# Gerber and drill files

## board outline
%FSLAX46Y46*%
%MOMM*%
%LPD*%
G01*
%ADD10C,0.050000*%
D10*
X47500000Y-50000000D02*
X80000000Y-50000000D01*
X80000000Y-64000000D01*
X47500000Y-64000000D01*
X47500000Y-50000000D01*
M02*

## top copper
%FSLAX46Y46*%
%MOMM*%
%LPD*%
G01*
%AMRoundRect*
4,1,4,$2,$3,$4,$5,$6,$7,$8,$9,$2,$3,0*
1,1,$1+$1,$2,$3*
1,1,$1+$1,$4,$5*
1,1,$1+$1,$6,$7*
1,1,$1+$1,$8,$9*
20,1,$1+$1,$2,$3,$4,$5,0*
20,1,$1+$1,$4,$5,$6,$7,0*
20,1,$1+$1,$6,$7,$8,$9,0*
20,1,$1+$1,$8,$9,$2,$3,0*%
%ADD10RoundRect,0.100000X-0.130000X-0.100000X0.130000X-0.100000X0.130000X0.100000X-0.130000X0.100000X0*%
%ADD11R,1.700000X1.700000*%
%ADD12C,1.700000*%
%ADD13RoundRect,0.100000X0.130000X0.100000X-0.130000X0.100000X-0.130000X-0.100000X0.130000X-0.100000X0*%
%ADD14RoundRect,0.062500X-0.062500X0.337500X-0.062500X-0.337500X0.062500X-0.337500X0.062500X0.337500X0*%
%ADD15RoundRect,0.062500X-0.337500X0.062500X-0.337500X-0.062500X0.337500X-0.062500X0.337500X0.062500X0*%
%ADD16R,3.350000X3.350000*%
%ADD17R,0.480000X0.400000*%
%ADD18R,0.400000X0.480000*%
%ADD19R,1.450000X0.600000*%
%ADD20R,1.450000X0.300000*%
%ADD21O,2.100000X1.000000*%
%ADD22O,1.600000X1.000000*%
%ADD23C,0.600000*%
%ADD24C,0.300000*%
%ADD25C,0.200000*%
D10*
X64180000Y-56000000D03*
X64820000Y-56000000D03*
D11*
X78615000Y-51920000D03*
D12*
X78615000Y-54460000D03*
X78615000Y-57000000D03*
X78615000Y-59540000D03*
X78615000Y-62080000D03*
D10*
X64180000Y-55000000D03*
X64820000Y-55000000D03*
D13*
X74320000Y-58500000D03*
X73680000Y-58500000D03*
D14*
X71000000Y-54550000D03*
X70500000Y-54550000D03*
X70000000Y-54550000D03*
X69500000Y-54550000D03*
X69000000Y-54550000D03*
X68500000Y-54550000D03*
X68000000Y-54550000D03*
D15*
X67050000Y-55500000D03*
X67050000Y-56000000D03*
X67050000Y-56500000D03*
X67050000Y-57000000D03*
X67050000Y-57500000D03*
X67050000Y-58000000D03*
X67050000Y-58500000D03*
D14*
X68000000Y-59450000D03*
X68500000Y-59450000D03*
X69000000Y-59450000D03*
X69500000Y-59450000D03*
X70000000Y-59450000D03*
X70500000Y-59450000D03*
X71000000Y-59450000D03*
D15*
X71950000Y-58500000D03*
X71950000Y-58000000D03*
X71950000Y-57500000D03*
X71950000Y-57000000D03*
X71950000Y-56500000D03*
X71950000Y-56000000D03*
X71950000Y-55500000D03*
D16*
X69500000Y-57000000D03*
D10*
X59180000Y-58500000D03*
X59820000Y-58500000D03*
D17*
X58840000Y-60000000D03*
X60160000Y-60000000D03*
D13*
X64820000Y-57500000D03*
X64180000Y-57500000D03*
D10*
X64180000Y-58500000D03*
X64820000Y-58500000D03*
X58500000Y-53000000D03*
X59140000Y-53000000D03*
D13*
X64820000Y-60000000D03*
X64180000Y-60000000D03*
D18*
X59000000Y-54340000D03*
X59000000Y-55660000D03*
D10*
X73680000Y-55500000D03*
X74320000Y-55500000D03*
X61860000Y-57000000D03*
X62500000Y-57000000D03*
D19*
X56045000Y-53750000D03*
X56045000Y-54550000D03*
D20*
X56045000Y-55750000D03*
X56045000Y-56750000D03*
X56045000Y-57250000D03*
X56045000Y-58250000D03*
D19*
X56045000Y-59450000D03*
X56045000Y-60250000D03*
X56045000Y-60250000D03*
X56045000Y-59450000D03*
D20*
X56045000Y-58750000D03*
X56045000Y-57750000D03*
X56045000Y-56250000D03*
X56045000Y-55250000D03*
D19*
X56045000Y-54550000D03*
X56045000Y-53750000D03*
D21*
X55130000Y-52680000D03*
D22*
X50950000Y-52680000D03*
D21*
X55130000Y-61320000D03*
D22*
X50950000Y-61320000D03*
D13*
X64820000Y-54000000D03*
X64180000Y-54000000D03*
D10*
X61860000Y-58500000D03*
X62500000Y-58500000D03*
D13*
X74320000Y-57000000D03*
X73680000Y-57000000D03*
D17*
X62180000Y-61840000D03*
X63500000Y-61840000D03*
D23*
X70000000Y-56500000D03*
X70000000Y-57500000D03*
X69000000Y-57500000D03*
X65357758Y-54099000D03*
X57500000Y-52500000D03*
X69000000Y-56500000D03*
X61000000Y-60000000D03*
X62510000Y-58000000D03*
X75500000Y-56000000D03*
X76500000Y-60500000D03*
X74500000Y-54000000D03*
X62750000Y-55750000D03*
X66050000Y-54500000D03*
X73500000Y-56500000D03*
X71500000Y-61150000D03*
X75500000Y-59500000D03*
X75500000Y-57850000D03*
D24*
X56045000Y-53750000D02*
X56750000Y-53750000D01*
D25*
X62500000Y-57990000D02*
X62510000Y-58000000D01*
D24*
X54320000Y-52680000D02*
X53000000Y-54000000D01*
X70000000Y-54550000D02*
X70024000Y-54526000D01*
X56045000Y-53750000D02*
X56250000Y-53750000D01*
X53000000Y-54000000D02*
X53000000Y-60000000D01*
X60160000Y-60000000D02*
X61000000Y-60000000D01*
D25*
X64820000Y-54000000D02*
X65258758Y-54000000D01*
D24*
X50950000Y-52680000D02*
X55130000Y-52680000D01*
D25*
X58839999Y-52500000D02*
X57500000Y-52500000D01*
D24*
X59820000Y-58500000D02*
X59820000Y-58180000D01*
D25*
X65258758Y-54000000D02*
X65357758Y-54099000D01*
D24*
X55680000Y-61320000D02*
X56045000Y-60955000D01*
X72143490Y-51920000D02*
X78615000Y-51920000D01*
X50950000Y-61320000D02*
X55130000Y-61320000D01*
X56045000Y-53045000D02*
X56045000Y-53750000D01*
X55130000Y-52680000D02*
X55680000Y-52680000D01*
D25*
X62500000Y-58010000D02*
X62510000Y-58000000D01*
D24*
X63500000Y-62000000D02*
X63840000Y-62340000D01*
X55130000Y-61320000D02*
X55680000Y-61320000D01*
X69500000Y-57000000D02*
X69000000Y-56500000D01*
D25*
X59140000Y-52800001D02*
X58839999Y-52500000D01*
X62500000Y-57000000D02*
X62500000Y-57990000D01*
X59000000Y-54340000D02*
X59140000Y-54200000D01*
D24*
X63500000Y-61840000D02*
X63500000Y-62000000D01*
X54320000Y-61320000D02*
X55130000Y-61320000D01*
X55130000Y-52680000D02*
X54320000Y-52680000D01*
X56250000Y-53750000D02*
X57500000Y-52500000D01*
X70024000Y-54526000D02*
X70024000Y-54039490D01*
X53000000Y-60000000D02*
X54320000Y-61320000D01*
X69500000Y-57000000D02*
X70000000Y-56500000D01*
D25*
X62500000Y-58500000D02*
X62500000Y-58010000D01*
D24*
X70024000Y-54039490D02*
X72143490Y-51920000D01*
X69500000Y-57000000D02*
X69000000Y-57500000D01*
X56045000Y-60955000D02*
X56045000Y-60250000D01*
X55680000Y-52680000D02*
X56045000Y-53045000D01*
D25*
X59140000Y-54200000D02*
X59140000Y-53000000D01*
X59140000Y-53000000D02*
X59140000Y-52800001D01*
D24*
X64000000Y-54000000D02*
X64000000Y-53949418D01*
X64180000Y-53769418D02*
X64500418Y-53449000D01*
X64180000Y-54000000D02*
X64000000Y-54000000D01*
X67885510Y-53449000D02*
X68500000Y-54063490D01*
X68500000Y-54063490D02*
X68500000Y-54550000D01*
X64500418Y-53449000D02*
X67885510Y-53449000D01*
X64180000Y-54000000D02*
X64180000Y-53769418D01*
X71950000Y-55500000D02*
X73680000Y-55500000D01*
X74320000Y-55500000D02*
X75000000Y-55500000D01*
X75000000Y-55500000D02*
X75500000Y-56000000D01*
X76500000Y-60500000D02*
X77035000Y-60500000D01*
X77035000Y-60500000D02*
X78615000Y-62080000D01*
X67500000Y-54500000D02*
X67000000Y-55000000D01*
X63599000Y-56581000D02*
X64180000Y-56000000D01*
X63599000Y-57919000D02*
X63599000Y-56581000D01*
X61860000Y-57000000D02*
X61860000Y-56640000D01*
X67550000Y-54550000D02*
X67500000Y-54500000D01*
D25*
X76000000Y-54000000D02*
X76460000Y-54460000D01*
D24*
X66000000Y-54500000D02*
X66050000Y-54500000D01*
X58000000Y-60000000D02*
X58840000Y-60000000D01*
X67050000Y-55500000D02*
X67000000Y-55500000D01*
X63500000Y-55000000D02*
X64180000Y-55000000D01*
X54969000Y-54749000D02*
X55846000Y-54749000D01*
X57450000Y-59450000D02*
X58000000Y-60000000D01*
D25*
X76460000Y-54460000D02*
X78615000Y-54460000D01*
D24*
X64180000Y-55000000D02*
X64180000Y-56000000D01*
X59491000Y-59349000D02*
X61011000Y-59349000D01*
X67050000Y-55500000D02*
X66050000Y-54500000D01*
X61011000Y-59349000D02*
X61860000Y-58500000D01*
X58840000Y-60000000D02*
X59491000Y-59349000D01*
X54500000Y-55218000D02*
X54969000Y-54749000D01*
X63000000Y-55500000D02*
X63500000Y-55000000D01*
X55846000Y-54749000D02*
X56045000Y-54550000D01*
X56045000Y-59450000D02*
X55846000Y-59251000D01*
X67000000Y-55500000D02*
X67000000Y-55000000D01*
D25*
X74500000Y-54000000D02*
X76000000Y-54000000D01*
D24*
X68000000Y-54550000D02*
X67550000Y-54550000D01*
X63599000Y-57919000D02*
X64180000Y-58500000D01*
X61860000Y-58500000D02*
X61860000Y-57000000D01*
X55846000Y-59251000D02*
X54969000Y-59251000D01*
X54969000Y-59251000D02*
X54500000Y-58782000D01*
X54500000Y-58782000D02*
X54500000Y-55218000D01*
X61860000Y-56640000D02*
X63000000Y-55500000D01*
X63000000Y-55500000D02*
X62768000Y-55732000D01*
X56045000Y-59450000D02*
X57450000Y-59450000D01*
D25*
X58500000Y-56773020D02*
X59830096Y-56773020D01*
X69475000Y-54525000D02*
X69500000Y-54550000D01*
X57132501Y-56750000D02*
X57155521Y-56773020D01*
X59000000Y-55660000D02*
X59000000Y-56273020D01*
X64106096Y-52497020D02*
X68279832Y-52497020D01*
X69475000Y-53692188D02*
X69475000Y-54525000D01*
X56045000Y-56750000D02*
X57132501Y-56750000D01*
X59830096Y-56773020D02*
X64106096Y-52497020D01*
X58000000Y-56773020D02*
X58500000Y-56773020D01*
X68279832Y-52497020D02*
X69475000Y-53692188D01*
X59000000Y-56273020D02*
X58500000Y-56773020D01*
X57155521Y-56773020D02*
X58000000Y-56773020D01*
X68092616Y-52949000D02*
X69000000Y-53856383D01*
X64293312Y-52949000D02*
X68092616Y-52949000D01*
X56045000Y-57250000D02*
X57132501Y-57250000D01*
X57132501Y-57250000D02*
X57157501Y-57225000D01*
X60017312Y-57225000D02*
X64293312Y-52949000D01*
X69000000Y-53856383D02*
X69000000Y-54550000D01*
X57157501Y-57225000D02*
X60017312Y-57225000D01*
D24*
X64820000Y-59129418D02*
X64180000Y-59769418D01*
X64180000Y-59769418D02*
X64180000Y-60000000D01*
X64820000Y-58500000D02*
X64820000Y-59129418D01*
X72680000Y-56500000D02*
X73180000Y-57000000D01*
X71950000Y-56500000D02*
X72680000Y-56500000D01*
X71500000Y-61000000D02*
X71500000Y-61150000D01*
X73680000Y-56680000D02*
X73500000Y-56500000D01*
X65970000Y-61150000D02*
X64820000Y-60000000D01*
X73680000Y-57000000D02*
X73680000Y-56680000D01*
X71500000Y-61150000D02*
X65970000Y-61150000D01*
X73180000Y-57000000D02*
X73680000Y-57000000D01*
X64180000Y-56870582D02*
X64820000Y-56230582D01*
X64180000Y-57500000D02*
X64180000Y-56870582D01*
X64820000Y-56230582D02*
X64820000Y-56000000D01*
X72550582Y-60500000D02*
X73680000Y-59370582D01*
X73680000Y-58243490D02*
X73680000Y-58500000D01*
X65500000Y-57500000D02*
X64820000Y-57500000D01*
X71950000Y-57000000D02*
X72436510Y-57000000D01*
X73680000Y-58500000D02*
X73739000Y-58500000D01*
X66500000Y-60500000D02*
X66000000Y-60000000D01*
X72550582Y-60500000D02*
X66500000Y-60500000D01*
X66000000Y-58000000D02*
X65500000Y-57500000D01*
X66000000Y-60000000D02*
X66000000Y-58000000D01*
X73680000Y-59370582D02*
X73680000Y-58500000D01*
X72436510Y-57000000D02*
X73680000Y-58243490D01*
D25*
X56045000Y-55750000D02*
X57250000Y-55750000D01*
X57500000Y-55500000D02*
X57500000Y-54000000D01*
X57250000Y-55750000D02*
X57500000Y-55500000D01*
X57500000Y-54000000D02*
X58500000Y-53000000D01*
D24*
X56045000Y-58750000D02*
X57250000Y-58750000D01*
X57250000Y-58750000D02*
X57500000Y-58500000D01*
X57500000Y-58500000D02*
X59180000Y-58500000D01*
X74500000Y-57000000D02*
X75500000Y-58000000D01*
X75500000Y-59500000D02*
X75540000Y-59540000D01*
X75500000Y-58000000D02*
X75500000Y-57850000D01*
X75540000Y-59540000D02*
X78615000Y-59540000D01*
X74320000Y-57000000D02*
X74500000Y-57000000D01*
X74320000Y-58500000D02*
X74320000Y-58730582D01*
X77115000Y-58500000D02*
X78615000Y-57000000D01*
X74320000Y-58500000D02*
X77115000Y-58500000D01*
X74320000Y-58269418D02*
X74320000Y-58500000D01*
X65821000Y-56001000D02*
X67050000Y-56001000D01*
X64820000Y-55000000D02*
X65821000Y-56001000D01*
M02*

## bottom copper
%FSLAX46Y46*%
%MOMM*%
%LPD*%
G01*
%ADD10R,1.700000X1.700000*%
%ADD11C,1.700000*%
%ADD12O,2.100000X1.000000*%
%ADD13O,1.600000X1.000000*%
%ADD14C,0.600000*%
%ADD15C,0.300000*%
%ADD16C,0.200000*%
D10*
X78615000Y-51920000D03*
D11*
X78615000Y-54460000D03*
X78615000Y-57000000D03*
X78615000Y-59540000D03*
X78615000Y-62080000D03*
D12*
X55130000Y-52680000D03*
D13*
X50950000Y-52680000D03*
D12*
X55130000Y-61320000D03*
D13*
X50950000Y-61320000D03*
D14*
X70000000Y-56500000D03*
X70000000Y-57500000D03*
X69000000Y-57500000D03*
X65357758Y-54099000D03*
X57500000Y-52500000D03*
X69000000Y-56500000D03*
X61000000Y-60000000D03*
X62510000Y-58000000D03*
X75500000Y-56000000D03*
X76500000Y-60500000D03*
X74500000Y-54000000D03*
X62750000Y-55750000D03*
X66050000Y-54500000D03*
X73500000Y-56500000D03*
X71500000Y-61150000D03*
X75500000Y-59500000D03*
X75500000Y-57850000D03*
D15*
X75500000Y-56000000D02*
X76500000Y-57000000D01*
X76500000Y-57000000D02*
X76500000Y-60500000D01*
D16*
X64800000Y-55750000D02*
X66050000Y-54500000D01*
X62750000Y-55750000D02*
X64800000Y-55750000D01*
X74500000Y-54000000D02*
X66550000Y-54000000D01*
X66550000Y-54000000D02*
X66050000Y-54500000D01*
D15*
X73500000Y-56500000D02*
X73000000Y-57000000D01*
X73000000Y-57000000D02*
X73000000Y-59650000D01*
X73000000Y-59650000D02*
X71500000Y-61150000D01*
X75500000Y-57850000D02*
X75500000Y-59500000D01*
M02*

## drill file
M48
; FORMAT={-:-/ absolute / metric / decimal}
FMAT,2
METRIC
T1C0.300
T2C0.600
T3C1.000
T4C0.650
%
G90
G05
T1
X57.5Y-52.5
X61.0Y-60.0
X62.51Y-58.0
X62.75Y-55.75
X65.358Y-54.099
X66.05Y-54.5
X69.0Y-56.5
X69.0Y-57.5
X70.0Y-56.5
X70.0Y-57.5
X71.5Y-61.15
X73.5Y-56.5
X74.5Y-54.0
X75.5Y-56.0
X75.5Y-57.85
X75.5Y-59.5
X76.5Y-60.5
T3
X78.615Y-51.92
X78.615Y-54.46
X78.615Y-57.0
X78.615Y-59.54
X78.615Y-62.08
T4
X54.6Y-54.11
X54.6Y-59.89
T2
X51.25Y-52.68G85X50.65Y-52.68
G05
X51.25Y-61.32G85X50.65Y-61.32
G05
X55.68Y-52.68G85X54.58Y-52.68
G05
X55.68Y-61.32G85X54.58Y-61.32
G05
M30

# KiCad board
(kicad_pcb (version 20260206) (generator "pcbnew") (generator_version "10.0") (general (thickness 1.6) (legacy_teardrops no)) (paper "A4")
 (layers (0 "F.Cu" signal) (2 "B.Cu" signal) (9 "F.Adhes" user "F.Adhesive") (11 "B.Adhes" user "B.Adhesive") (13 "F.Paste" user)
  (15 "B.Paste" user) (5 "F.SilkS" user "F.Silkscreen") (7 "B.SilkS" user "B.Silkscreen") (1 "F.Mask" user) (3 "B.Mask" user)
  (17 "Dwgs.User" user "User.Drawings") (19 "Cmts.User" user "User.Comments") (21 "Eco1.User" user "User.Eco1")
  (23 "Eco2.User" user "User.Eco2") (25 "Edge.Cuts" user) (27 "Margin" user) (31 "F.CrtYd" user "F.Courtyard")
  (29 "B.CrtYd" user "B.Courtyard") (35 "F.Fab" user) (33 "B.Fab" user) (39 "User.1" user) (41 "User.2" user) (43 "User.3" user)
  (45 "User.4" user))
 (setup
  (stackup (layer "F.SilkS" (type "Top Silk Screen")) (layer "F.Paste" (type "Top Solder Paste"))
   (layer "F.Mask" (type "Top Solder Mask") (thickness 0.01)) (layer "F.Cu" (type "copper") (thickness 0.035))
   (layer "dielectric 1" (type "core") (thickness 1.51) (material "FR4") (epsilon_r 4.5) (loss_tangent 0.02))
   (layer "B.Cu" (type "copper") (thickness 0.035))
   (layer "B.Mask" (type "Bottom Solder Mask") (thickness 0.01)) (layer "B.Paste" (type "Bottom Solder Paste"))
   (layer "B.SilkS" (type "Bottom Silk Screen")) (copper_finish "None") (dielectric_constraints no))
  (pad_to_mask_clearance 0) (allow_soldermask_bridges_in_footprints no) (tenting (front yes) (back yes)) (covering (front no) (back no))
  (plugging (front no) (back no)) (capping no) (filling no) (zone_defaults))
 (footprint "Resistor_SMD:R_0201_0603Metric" (layer "F.Cu") (at 64.5 56)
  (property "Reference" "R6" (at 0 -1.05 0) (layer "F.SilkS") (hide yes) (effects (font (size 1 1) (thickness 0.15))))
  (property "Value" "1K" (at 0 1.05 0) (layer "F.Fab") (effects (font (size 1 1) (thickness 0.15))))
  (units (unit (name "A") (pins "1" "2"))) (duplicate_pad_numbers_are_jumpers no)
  (pad "" smd roundrect (at -0.345 0) (size 0.318 0.36) (layers "F.Paste") (roundrect_rratio 0.25))
  (pad "" smd roundrect (at 0.345 0) (size 0.318 0.36) (layers "F.Paste") (roundrect_rratio 0.25))
  (pad "1" smd roundrect (at -0.32 0) (size 0.46 0.4) (layers "F.Cu" "F.Mask") (roundrect_rratio 0.25) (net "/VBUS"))
  (pad "2" smd roundrect (at 0.32 0) (size 0.46 0.4) (layers "F.Cu" "F.Mask") (roundrect_rratio 0.25) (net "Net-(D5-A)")))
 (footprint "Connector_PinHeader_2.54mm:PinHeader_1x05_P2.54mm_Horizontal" (layer "F.Cu") (at 78.615 51.92)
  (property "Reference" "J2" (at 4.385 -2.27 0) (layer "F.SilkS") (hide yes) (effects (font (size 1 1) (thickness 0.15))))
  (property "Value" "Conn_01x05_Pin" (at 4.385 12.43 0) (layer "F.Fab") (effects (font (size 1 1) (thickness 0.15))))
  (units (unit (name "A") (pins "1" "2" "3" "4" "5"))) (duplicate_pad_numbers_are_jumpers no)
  (pad "1" thru_hole rect (at 0 0) (size 1.7 1.7) (drill 1) (layers "*.Cu" "*.Mask") (remove_unused_layers no) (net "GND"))
  (pad "2" thru_hole circle (at 0 2.54) (size 1.7 1.7) (drill 1) (layers "*.Cu" "*.Mask") (remove_unused_layers no) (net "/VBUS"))
  (pad "3" thru_hole circle (at 0 5.08) (size 1.7 1.7) (drill 1) (layers "*.Cu" "*.Mask") (remove_unused_layers no) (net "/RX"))
  (pad "4" thru_hole circle (at 0 7.62) (size 1.7 1.7) (drill 1) (layers "*.Cu" "*.Mask") (remove_unused_layers no) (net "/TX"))
  (pad "5" thru_hole circle (at 0 10.16) (size 1.7 1.7) (drill 1) (layers "*.Cu" "*.Mask") (remove_unused_layers no) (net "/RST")))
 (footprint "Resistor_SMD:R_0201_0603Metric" (layer "F.Cu") (at 64.5 55)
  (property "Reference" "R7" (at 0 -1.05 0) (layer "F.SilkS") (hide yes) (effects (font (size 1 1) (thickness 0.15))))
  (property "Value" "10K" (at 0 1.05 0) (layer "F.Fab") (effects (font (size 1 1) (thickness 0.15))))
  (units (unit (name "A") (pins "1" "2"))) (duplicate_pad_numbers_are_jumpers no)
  (pad "" smd roundrect (at -0.345 0) (size 0.318 0.36) (layers "F.Paste") (roundrect_rratio 0.25))
  (pad "" smd roundrect (at 0.345 0) (size 0.318 0.36) (layers "F.Paste") (roundrect_rratio 0.25))
  (pad "1" smd roundrect (at -0.32 0) (size 0.46 0.4) (layers "F.Cu" "F.Mask") (roundrect_rratio 0.25) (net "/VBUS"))
  (pad "2" smd roundrect (at 0.32 0) (size 0.46 0.4) (layers "F.Cu" "F.Mask") (roundrect_rratio 0.25) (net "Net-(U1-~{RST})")))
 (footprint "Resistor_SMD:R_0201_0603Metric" (layer "F.Cu") (at 74 58.5 180)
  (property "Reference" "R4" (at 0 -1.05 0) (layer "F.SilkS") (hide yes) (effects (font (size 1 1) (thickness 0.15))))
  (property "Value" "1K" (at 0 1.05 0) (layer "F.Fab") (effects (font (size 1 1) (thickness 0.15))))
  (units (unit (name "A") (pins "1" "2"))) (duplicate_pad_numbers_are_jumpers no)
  (pad "" smd roundrect (at -0.345 0 180) (size 0.318 0.36) (layers "F.Paste") (roundrect_rratio 0.25))
  (pad "" smd roundrect (at 0.345 0 180) (size 0.318 0.36) (layers "F.Paste") (roundrect_rratio 0.25))
  (pad "1" smd roundrect (at -0.32 0 180) (size 0.46 0.4) (layers "F.Cu" "F.Mask") (roundrect_rratio 0.25) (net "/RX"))
  (pad "2" smd roundrect (at 0.32 0 180) (size 0.46 0.4) (layers "F.Cu" "F.Mask") (roundrect_rratio 0.25) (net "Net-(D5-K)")))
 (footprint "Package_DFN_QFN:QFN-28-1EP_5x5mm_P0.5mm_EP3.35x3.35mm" (layer "F.Cu") (at 69.5 57 -90)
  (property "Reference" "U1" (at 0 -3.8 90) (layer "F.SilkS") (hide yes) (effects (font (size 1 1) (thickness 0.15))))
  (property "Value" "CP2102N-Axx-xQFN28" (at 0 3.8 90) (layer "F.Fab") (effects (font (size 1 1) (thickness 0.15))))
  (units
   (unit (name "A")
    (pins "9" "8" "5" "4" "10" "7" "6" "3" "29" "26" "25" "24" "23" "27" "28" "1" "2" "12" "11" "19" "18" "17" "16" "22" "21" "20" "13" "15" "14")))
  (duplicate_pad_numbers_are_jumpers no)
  (pad "" smd roundrect (at -1.12 -1.12 270) (size 0.9 0.9) (layers "F.Paste") (roundrect_rratio 0.25))
  (pad "" smd roundrect (at -1.12 0 270) (size 0.9 0.9) (layers "F.Paste") (roundrect_rratio 0.25))
  (pad "" smd roundrect (at -1.12 1.12 270) (size 0.9 0.9) (layers "F.Paste") (roundrect_rratio 0.25))
  (pad "" smd roundrect (at 0 -1.12 270) (size 0.9 0.9) (layers "F.Paste") (roundrect_rratio 0.25))
  (pad "" smd roundrect (at 0 0 270) (size 0.9 0.9) (layers "F.Paste") (roundrect_rratio 0.25))
  (pad "" smd roundrect (at 0 1.12 270) (size 0.9 0.9) (layers "F.Paste") (roundrect_rratio 0.25))
  (pad "" smd roundrect (at 1.12 -1.12 270) (size 0.9 0.9) (layers "F.Paste") (roundrect_rratio 0.25))
  (pad "" smd roundrect (at 1.12 0 270) (size 0.9 0.9) (layers "F.Paste") (roundrect_rratio 0.25))
  (pad "" smd roundrect (at 1.12 1.12 270) (size 0.9 0.9) (layers "F.Paste") (roundrect_rratio 0.25))
  (pad "1" smd roundrect (at -2.45 -1.5 270) (size 0.8 0.25) (layers "F.Cu" "F.Mask" "F.Paste") (roundrect_rratio 0.25)
   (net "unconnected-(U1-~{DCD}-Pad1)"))
  (pad "2" smd roundrect (at -2.45 -1 270) (size 0.8 0.25) (layers "F.Cu" "F.Mask" "F.Paste") (roundrect_rratio 0.25)
   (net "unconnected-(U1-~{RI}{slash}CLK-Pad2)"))
  (pad "3" smd roundrect (at -2.45 -0.5 270) (size 0.8 0.25) (layers "F.Cu" "F.Mask" "F.Paste") (roundrect_rratio 0.25) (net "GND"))
  (pad "4" smd roundrect (at -2.45 0 270) (size 0.8 0.25) (layers "F.Cu" "F.Mask" "F.Paste") (roundrect_rratio 0.25) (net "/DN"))
  (pad "5" smd roundrect (at -2.45 0.5 270) (size 0.8 0.25) (layers "F.Cu" "F.Mask" "F.Paste") (roundrect_rratio 0.25) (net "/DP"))
  (pad "6" smd roundrect (at -2.45 1 270) (size 0.8 0.25) (layers "F.Cu" "F.Mask" "F.Paste") (roundrect_rratio 0.25) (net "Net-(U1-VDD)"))
  (pad "7" smd roundrect (at -2.45 1.5 270) (size 0.8 0.25) (layers "F.Cu" "F.Mask" "F.Paste") (roundrect_rratio 0.25) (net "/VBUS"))
  (pad "8" smd roundrect (at -1.5 2.45 270) (size 0.25 0.8) (layers "F.Cu" "F.Mask" "F.Paste") (roundrect_rratio 0.25) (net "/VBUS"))
  (pad "9" smd roundrect (at -1 2.45 270) (size 0.25 0.8) (layers "F.Cu" "F.Mask" "F.Paste") (roundrect_rratio 0.25) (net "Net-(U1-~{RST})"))
  (pad "10" smd roundrect (at -0.5 2.45 270) (size 0.25 0.8) (layers "F.Cu" "F.Mask" "F.Paste") (roundrect_rratio 0.25)
   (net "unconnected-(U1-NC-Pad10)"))
  (pad "11" smd roundrect (at 0 2.45 270) (size 0.25 0.8) (layers "F.Cu" "F.Mask" "F.Paste") (roundrect_rratio 0.25)
   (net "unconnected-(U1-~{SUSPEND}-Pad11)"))
  (pad "12" smd roundrect (at 0.5 2.45 270) (size 0.25 0.8) (layers "F.Cu" "F.Mask" "F.Paste") (roundrect_rratio 0.25)
   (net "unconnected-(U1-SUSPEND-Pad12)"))
  (pad "13" smd roundrect (at 1 2.45 270) (size 0.25 0.8) (layers "F.Cu" "F.Mask" "F.Paste") (roundrect_rratio 0.25)
   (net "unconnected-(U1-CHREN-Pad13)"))
  (pad "14" smd roundrect (at 1.5 2.45 270) (size 0.25 0.8) (layers "F.Cu" "F.Mask" "F.Paste") (roundrect_rratio 0.25)
   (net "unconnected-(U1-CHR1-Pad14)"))
  (pad "15" smd roundrect (at 2.45 1.5 270) (size 0.8 0.25) (layers "F.Cu" "F.Mask" "F.Paste") (roundrect_rratio 0.25)
   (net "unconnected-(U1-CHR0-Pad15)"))
  (pad "16" smd roundrect (at 2.45 1 270) (size 0.8 0.25) (layers "F.Cu" "F.Mask" "F.Paste") (roundrect_rratio 0.25)
   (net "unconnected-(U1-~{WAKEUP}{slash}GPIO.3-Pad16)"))
  (pad "17" smd roundrect (at 2.45 0.5 270) (size 0.8 0.25) (layers "F.Cu" "F.Mask" "F.Paste") (roundrect_rratio 0.25)
   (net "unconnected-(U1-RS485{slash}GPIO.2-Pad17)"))
  (pad "18" smd roundrect (at 2.45 0 270) (size 0.8 0.25) (layers "F.Cu" "F.Mask" "F.Paste") (roundrect_rratio 0.25)
   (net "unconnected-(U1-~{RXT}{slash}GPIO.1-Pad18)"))
  (pad "19" smd roundrect (at 2.45 -0.5 270) (size 0.8 0.25) (layers "F.Cu" "F.Mask" "F.Paste") (roundrect_rratio 0.25)
   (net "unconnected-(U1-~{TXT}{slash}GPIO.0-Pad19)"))
  (pad "20" smd roundrect (at 2.45 -1 270) (size 0.8 0.25) (layers "F.Cu" "F.Mask" "F.Paste") (roundrect_rratio 0.25)
   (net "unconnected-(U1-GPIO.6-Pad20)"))
  (pad "21" smd roundrect (at 2.45 -1.5 270) (size 0.8 0.25) (layers "F.Cu" "F.Mask" "F.Paste") (roundrect_rratio 0.25)
   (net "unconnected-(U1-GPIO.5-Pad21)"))
  (pad "22" smd roundrect (at 1.5 -2.45 270) (size 0.25 0.8) (layers "F.Cu" "F.Mask" "F.Paste") (roundrect_rratio 0.25)
   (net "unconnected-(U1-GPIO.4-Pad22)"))
  (pad "23" smd roundrect (at 1 -2.45 270) (size 0.25 0.8) (layers "F.Cu" "F.Mask" "F.Paste") (roundrect_rratio 0.25)
   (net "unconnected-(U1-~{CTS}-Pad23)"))
  (pad "24" smd roundrect (at 0.5 -2.45 270) (size 0.25 0.8) (layers "F.Cu" "F.Mask" "F.Paste") (roundrect_rratio 0.25)
   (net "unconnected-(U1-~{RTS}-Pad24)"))
  (pad "25" smd roundrect (at 0 -2.45 270) (size 0.25 0.8) (layers "F.Cu" "F.Mask" "F.Paste") (roundrect_rratio 0.25) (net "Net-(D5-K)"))
  (pad "26" smd roundrect (at -0.5 -2.45 270) (size 0.25 0.8) (layers "F.Cu" "F.Mask" "F.Paste") (roundrect_rratio 0.25) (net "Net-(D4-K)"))
  (pad "27" smd roundrect (at -1 -2.45 270) (size 0.25 0.8) (layers "F.Cu" "F.Mask" "F.Paste") (roundrect_rratio 0.25)
   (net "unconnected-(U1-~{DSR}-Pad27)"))
  (pad "28" smd roundrect (at -1.5 -2.45 270) (size 0.25 0.8) (layers "F.Cu" "F.Mask" "F.Paste") (roundrect_rratio 0.25)
   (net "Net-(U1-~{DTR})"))
  (pad "29" smd rect (at 0 0 270) (size 3.35 3.35) (layers "F.Cu" "F.Mask") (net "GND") (zone_connect 2)))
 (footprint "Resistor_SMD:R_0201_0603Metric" (layer "F.Cu") (at 59.5 58.5)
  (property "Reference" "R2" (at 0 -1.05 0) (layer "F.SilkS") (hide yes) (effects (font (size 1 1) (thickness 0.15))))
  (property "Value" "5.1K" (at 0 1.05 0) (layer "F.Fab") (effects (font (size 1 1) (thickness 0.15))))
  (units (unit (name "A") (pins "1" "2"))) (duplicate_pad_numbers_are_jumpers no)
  (pad "" smd roundrect (at -0.345 0) (size 0.318 0.36) (layers "F.Paste") (roundrect_rratio 0.25))
  (pad "" smd roundrect (at 0.345 0) (size 0.318 0.36) (layers "F.Paste") (roundrect_rratio 0.25))
  (pad "1" smd roundrect (at -0.32 0) (size 0.46 0.4) (layers "F.Cu" "F.Mask") (roundrect_rratio 0.25) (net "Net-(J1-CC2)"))
  (pad "2" smd roundrect (at 0.32 0) (size 0.46 0.4) (layers "F.Cu" "F.Mask") (roundrect_rratio 0.25) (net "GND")))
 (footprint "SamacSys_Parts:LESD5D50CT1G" (layer "F.Cu") (at 59.5 60)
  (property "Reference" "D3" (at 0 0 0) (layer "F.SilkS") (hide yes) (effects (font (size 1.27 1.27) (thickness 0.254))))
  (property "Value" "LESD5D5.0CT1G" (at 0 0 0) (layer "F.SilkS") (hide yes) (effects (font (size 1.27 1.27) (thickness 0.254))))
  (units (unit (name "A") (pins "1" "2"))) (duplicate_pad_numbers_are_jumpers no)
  (pad "1" smd rect (at -0.66 0 90) (size 0.4 0.48) (layers "F.Cu" "F.Mask" "F.Paste") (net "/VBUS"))
  (pad "2" smd rect (at 0.66 0 90) (size 0.4 0.48) (layers "F.Cu" "F.Mask" "F.Paste") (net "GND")))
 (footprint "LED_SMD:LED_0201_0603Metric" (layer "F.Cu") (at 64.5 57.5 180)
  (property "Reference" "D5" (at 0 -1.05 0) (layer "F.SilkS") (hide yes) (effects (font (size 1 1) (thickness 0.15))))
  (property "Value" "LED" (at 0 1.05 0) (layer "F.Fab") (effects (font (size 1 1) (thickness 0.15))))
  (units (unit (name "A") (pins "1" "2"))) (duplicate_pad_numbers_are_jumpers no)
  (pad "" smd roundrect (at -0.345 0 180) (size 0.318 0.36) (layers "F.Paste") (roundrect_rratio 0.25))
  (pad "" smd roundrect (at 0.345 0 180) (size 0.318 0.36) (layers "F.Paste") (roundrect_rratio 0.25))
  (pad "1" smd roundrect (at -0.32 0 180) (size 0.46 0.4) (layers "F.Cu" "F.Mask") (roundrect_rratio 0.25) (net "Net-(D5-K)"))
  (pad "2" smd roundrect (at 0.32 0 180) (size 0.46 0.4) (layers "F.Cu" "F.Mask") (roundrect_rratio 0.25) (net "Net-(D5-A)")))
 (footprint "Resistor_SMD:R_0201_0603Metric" (layer "F.Cu") (at 64.5 58.5)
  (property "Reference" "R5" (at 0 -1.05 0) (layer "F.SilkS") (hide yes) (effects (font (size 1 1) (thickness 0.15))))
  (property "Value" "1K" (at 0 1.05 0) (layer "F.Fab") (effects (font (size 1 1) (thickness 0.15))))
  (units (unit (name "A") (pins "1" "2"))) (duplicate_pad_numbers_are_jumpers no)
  (pad "" smd roundrect (at -0.345 0) (size 0.318 0.36) (layers "F.Paste") (roundrect_rratio 0.25))
  (pad "" smd roundrect (at 0.345 0) (size 0.318 0.36) (layers "F.Paste") (roundrect_rratio 0.25))
  (pad "1" smd roundrect (at -0.32 0) (size 0.46 0.4) (layers "F.Cu" "F.Mask") (roundrect_rratio 0.25) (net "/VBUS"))
  (pad "2" smd roundrect (at 0.32 0) (size 0.46 0.4) (layers "F.Cu" "F.Mask") (roundrect_rratio 0.25) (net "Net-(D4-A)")))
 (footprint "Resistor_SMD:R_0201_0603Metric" (layer "F.Cu") (at 58.82 53)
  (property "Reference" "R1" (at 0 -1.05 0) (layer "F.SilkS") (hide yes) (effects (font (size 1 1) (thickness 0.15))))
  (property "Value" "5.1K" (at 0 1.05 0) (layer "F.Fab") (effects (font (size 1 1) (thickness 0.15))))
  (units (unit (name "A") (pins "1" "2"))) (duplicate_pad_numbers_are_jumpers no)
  (pad "" smd roundrect (at -0.345 0) (size 0.318 0.36) (layers "F.Paste") (roundrect_rratio 0.25))
  (pad "" smd roundrect (at 0.345 0) (size 0.318 0.36) (layers "F.Paste") (roundrect_rratio 0.25))
  (pad "1" smd roundrect (at -0.32 0) (size 0.46 0.4) (layers "F.Cu" "F.Mask") (roundrect_rratio 0.25) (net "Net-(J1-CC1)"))
  (pad "2" smd roundrect (at 0.32 0) (size 0.46 0.4) (layers "F.Cu" "F.Mask") (roundrect_rratio 0.25) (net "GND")))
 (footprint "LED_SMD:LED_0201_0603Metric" (layer "F.Cu") (at 64.5 60 180)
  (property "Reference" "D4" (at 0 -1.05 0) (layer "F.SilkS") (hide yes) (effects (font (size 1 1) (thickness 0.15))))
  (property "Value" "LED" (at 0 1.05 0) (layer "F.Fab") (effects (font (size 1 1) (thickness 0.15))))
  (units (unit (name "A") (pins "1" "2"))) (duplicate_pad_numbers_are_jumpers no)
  (pad "" smd roundrect (at -0.345 0 180) (size 0.318 0.36) (layers "F.Paste") (roundrect_rratio 0.25))
  (pad "" smd roundrect (at 0.345 0 180) (size 0.318 0.36) (layers "F.Paste") (roundrect_rratio 0.25))
  (pad "1" smd roundrect (at -0.32 0 180) (size 0.46 0.4) (layers "F.Cu" "F.Mask") (roundrect_rratio 0.25) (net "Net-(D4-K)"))
  (pad "2" smd roundrect (at 0.32 0 180) (size 0.46 0.4) (layers "F.Cu" "F.Mask") (roundrect_rratio 0.25) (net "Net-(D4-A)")))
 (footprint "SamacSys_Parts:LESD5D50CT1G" (layer "F.Cu") (at 59 55 -90)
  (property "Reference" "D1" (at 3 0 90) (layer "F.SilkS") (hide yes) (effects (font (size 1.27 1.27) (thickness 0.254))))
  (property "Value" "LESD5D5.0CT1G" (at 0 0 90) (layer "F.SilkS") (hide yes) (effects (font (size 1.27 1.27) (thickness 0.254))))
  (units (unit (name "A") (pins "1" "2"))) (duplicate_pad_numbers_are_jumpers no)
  (pad "1" smd rect (at -0.66 0) (size 0.4 0.48) (layers "F.Cu" "F.Mask" "F.Paste") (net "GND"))
  (pad "2" smd rect (at 0.66 0) (size 0.4 0.48) (layers "F.Cu" "F.Mask" "F.Paste") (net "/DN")))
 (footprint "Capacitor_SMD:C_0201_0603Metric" (layer "F.Cu") (at 74 55.5)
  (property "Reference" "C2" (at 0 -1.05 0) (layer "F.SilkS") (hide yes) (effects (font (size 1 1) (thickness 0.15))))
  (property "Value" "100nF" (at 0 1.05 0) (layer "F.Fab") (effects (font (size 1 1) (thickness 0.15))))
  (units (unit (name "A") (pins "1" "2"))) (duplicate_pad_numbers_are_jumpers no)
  (pad "" smd roundrect (at -0.345 0) (size 0.318 0.36) (layers "F.Paste") (roundrect_rratio 0.25))
  (pad "" smd roundrect (at 0.345 0) (size 0.318 0.36) (layers "F.Paste") (roundrect_rratio 0.25))
  (pad "1" smd roundrect (at -0.32 0) (size 0.46 0.4) (layers "F.Cu" "F.Mask") (roundrect_rratio 0.25) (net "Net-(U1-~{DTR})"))
  (pad "2" smd roundrect (at 0.32 0) (size 0.46 0.4) (layers "F.Cu" "F.Mask") (roundrect_rratio 0.25) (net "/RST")))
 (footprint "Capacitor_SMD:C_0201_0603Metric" (layer "F.Cu") (at 62.18 57)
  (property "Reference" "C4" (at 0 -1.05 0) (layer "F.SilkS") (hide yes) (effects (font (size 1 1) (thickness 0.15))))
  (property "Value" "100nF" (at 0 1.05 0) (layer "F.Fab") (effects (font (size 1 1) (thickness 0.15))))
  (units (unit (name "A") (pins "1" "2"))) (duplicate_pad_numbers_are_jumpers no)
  (pad "" smd roundrect (at -0.345 0) (size 0.318 0.36) (layers "F.Paste") (roundrect_rratio 0.25))
  (pad "" smd roundrect (at 0.345 0) (size 0.318 0.36) (layers "F.Paste") (roundrect_rratio 0.25))
  (pad "1" smd roundrect (at -0.32 0) (size 0.46 0.4) (layers "F.Cu" "F.Mask") (roundrect_rratio 0.25) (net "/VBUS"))
  (pad "2" smd roundrect (at 0.32 0) (size 0.46 0.4) (layers "F.Cu" "F.Mask") (roundrect_rratio 0.25) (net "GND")))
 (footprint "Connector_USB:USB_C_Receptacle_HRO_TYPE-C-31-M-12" (layer "F.Cu") (at 52 57 -90)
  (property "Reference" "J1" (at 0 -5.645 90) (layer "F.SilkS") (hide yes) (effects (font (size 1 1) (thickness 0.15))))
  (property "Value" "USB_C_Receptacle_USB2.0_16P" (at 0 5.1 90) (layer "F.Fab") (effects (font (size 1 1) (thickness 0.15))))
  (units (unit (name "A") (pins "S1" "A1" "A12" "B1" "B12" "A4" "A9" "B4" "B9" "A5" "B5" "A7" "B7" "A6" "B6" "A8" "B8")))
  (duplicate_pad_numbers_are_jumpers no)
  (pad "" np_thru_hole circle (at -2.89 -2.6 270) (size 0.65 0.65) (drill 0.65) (layers "*.Cu" "*.Mask"))
  (pad "" np_thru_hole circle (at 2.89 -2.6 270) (size 0.65 0.65) (drill 0.65) (layers "*.Cu" "*.Mask"))
  (pad "A1" smd rect (at -3.25 -4.045 270) (size 0.6 1.45) (layers "F.Cu" "F.Mask" "F.Paste") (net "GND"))
  (pad "A4" smd rect (at -2.45 -4.045 270) (size 0.6 1.45) (layers "F.Cu" "F.Mask" "F.Paste") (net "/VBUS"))
  (pad "A5" smd rect (at -1.25 -4.045 270) (size 0.3 1.45) (layers "F.Cu" "F.Mask" "F.Paste") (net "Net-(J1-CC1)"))
  (pad "A6" smd rect (at -0.25 -4.045 270) (size 0.3 1.45) (layers "F.Cu" "F.Mask" "F.Paste") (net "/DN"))
  (pad "A7" smd rect (at 0.25 -4.045 270) (size 0.3 1.45) (layers "F.Cu" "F.Mask" "F.Paste") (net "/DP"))
  (pad "A8" smd rect (at 1.25 -4.045 270) (size 0.3 1.45) (layers "F.Cu" "F.Mask" "F.Paste") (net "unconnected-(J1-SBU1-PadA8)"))
  (pad "A9" smd rect (at 2.45 -4.045 270) (size 0.6 1.45) (layers "F.Cu" "F.Mask" "F.Paste") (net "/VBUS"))
  (pad "A12" smd rect (at 3.25 -4.045 270) (size 0.6 1.45) (layers "F.Cu" "F.Mask" "F.Paste") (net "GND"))
  (pad "B1" smd rect (at 3.25 -4.045 270) (size 0.6 1.45) (layers "F.Cu" "F.Mask" "F.Paste") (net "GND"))
  (pad "B4" smd rect (at 2.45 -4.045 270) (size 0.6 1.45) (layers "F.Cu" "F.Mask" "F.Paste") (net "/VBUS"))
  (pad "B5" smd rect (at 1.75 -4.045 270) (size 0.3 1.45) (layers "F.Cu" "F.Mask" "F.Paste") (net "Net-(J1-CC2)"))
  (pad "B6" smd rect (at 0.75 -4.045 270) (size 0.3 1.45) (layers "F.Cu" "F.Mask" "F.Paste") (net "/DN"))
  (pad "B7" smd rect (at -0.75 -4.045 270) (size 0.3 1.45) (layers "F.Cu" "F.Mask" "F.Paste") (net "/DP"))
  (pad "B8" smd rect (at -1.75 -4.045 270) (size 0.3 1.45) (layers "F.Cu" "F.Mask" "F.Paste") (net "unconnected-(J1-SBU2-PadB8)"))
  (pad "B9" smd rect (at -2.45 -4.045 270) (size 0.6 1.45) (layers "F.Cu" "F.Mask" "F.Paste") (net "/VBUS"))
  (pad "B12" smd rect (at -3.25 -4.045 270) (size 0.6 1.45) (layers "F.Cu" "F.Mask" "F.Paste") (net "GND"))
  (pad "S1" thru_hole oval (at -4.32 -3.13 270) (size 1 2.1) (drill oval 0.6 1.7) (layers "*.Cu" "*.Mask") (remove_unused_layers no)
   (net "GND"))
  (pad "S1" thru_hole oval (at -4.32 1.05 270) (size 1 1.6) (drill oval 0.6 1.2) (layers "*.Cu" "*.Mask") (remove_unused_layers no)
   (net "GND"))
  (pad "S1" thru_hole oval (at 4.32 -3.13 270) (size 1 2.1) (drill oval 0.6 1.7) (layers "*.Cu" "*.Mask") (remove_unused_layers no)
   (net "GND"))
  (pad "S1" thru_hole oval (at 4.32 1.05 270) (size 1 1.6) (drill oval 0.6 1.2) (layers "*.Cu" "*.Mask") (remove_unused_layers no)
   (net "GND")))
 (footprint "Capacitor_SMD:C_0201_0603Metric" (layer "F.Cu") (at 64.5 54 180)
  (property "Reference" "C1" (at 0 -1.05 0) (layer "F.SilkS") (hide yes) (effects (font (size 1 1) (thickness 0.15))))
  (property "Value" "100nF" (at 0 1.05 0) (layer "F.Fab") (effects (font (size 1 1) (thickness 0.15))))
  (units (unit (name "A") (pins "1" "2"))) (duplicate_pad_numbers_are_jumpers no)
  (pad "" smd roundrect (at -0.345 0 180) (size 0.318 0.36) (layers "F.Paste") (roundrect_rratio 0.25))
  (pad "" smd roundrect (at 0.345 0 180) (size 0.318 0.36) (layers "F.Paste") (roundrect_rratio 0.25))
  (pad "1" smd roundrect (at -0.32 0 180) (size 0.46 0.4) (layers "F.Cu" "F.Mask") (roundrect_rratio 0.25) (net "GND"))
  (pad "2" smd roundrect (at 0.32 0 180) (size 0.46 0.4) (layers "F.Cu" "F.Mask") (roundrect_rratio 0.25) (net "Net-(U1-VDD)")))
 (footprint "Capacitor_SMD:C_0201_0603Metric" (layer "F.Cu") (at 62.18 58.5)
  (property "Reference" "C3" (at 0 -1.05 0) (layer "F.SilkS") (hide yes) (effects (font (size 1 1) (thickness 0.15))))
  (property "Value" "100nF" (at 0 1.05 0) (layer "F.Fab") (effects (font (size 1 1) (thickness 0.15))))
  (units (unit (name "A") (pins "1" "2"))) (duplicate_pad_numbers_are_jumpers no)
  (pad "" smd roundrect (at -0.345 0) (size 0.318 0.36) (layers "F.Paste") (roundrect_rratio 0.25))
  (pad "" smd roundrect (at 0.345 0) (size 0.318 0.36) (layers "F.Paste") (roundrect_rratio 0.25))
  (pad "1" smd roundrect (at -0.32 0) (size 0.46 0.4) (layers "F.Cu" "F.Mask") (roundrect_rratio 0.25) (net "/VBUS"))
  (pad "2" smd roundrect (at 0.32 0) (size 0.46 0.4) (layers "F.Cu" "F.Mask") (roundrect_rratio 0.25) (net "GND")))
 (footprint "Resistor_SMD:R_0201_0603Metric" (layer "F.Cu") (at 74 57 180)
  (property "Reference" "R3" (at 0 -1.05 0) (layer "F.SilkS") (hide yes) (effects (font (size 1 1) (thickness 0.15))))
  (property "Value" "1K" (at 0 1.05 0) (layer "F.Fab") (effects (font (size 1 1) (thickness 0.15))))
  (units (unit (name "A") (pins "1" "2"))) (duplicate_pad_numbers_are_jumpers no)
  (pad "" smd roundrect (at -0.345 0 180) (size 0.318 0.36) (layers "F.Paste") (roundrect_rratio 0.25))
  (pad "" smd roundrect (at 0.345 0 180) (size 0.318 0.36) (layers "F.Paste") (roundrect_rratio 0.25))
  (pad "1" smd roundrect (at -0.32 0 180) (size 0.46 0.4) (layers "F.Cu" "F.Mask") (roundrect_rratio 0.25) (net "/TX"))
  (pad "2" smd roundrect (at 0.32 0 180) (size 0.46 0.4) (layers "F.Cu" "F.Mask") (roundrect_rratio 0.25) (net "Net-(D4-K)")))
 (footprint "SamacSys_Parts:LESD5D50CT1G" (layer "F.Cu") (at 62.84 61.84)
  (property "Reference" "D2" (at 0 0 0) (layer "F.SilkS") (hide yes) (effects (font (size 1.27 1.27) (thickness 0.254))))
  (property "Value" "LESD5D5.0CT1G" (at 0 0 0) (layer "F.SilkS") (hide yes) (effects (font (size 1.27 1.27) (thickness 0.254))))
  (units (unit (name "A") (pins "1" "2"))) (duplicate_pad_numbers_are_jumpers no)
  (pad "1" smd rect (at -0.66 0 90) (size 0.4 0.48) (layers "F.Cu" "F.Mask" "F.Paste") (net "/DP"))
  (pad "2" smd rect (at 0.66 0 90) (size 0.4 0.48) (layers "F.Cu" "F.Mask" "F.Paste") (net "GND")))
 (gr_rect (start 47.5 50) (end 80 64) (stroke (width 0.05) (type default)) (fill no) (layer "Edge.Cuts"))
 (segment (start 56.045 53.75) (end 56.75 53.75) (width 0.3) (layer "F.Cu") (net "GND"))
 (segment (start 62.5 57.99) (end 62.51 58) (width 0.2) (layer "F.Cu") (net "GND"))
 (segment (start 54.32 52.68) (end 53 54) (width 0.3) (layer "F.Cu") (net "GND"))
 (segment (start 70 54.55) (end 70.024 54.526) (width 0.3) (layer "F.Cu") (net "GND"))
 (segment (start 56.045 53.75) (end 56.25 53.75) (width 0.3) (layer "F.Cu") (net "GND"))
 (segment (start 53 54) (end 53 60) (width 0.3) (layer "F.Cu") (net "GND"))
 (segment (start 60.16 60) (end 61 60) (width 0.3) (layer "F.Cu") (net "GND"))
 (segment (start 64.82 54) (end 65.258758 54) (width 0.2) (layer "F.Cu") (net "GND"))
 (segment (start 50.95 52.68) (end 55.13 52.68) (width 0.3) (layer "F.Cu") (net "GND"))
 (segment (start 58.839999 52.5) (end 57.5 52.5) (width 0.2) (layer "F.Cu") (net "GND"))
 (segment (start 59.82 58.5) (end 59.82 58.18) (width 0.3) (layer "F.Cu") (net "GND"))
 (segment (start 65.258758 54) (end 65.357758 54.099) (width 0.2) (layer "F.Cu") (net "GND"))
 (segment (start 55.68 61.32) (end 56.045 60.955) (width 0.3) (layer "F.Cu") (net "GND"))
 (segment (start 72.14349 51.92) (end 78.615 51.92) (width 0.3) (layer "F.Cu") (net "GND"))
 (segment (start 50.95 61.32) (end 55.13 61.32) (width 0.3) (layer "F.Cu") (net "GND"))
 (segment (start 56.045 53.045) (end 56.045 53.75) (width 0.3) (layer "F.Cu") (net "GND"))
 (segment (start 55.13 52.68) (end 55.68 52.68) (width 0.3) (layer "F.Cu") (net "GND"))
 (segment (start 62.5 58.01) (end 62.51 58) (width 0.2) (layer "F.Cu") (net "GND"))
 (segment (start 63.5 62) (end 63.84 62.34) (width 0.3) (layer "F.Cu") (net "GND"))
 (segment (start 55.13 61.32) (end 55.68 61.32) (width 0.3) (layer "F.Cu") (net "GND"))
 (segment (start 69.5 57) (end 69 56.5) (width 0.3) (layer "F.Cu") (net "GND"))
 (segment (start 59.14 52.800001) (end 58.839999 52.5) (width 0.2) (layer "F.Cu") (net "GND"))
 (segment (start 62.5 57) (end 62.5 57.99) (width 0.2) (layer "F.Cu") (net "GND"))
 (segment (start 59 54.34) (end 59.14 54.2) (width 0.2) (layer "F.Cu") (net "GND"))
 (segment (start 63.5 61.84) (end 63.5 62) (width 0.3) (layer "F.Cu") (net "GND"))
 (segment (start 54.32 61.32) (end 55.13 61.32) (width 0.3) (layer "F.Cu") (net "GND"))
 (segment (start 55.13 52.68) (end 54.32 52.68) (width 0.3) (layer "F.Cu") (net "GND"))
 (segment (start 56.25 53.75) (end 57.5 52.5) (width 0.3) (layer "F.Cu") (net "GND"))
 (segment (start 70.024 54.526) (end 70.024 54.03949) (width 0.3) (layer "F.Cu") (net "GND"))
 (segment (start 53 60) (end 54.32 61.32) (width 0.3) (layer "F.Cu") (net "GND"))
 (segment (start 69.5 57) (end 70 56.5) (width 0.3) (layer "F.Cu") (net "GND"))
 (segment (start 62.5 58.5) (end 62.5 58.01) (width 0.2) (layer "F.Cu") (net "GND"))
 (segment (start 70.024 54.03949) (end 72.14349 51.92) (width 0.3) (layer "F.Cu") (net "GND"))
 (segment (start 69.5 57) (end 69 57.5) (width 0.3) (layer "F.Cu") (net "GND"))
 (segment (start 56.045 60.955) (end 56.045 60.25) (width 0.3) (layer "F.Cu") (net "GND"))
 (segment (start 55.68 52.68) (end 56.045 53.045) (width 0.3) (layer "F.Cu") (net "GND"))
 (segment (start 59.14 54.2) (end 59.14 53) (width 0.2) (layer "F.Cu") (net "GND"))
 (segment (start 59.14 53) (end 59.14 52.800001) (width 0.2) (layer "F.Cu") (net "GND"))
 (via (at 70 56.5) (size 0.6) (drill 0.3) (layers "F.Cu" "B.Cu") (capping no) (covering (front no) (back no))
  (plugging (front no) (back no)) (filling no) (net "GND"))
 (via (at 70 57.5) (size 0.6) (drill 0.3) (layers "F.Cu" "B.Cu") (capping no) (covering (front no) (back no))
  (plugging (front no) (back no)) (filling no) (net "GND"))
 (via (at 69 57.5) (size 0.6) (drill 0.3) (layers "F.Cu" "B.Cu") (capping no) (covering (front no) (back no))
  (plugging (front no) (back no)) (filling no) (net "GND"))
 (via (at 65.357758 54.099) (size 0.6) (drill 0.3) (layers "F.Cu" "B.Cu") (capping no) (covering (front no) (back no))
  (plugging (front no) (back no)) (filling no) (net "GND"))
 (via (at 57.5 52.5) (size 0.6) (drill 0.3) (layers "F.Cu" "B.Cu") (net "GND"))
 (via (at 69 56.5) (size 0.6) (drill 0.3) (layers "F.Cu" "B.Cu") (capping no) (covering (front no) (back no))
  (plugging (front no) (back no)) (filling no) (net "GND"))
 (via (at 61 60) (size 0.6) (drill 0.3) (layers "F.Cu" "B.Cu") (capping no) (covering (front no) (back no)) (plugging (front no) (back no))
  (filling no) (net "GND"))
 (via (at 62.51 58) (size 0.6) (drill 0.3) (layers "F.Cu" "B.Cu") (capping no) (covering (front no) (back no))
  (plugging (front no) (back no)) (filling no) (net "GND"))
 (segment (start 64 54) (end 64 53.949418) (width 0.3) (layer "F.Cu") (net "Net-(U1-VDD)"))
 (segment (start 64.18 53.769418) (end 64.500418 53.449) (width 0.3) (layer "F.Cu") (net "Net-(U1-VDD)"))
 (segment (start 64.18 54) (end 64 54) (width 0.3) (layer "F.Cu") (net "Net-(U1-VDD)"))
 (segment (start 67.88551 53.449) (end 68.5 54.06349) (width 0.3) (layer "F.Cu") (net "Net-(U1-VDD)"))
 (segment (start 68.5 54.06349) (end 68.5 54.55) (width 0.3) (layer "F.Cu") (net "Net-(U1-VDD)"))
 (segment (start 64.500418 53.449) (end 67.88551 53.449) (width 0.3) (layer "F.Cu") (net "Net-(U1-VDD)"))
 (segment (start 64.18 54) (end 64.18 53.769418) (width 0.3) (layer "F.Cu") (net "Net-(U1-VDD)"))
 (segment (start 71.95 55.5) (end 73.68 55.5) (width 0.3) (layer "F.Cu") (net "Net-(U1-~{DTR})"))
 (segment (start 74.32 55.5) (end 75 55.5) (width 0.3) (layer "F.Cu") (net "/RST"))
 (segment (start 75 55.5) (end 75.5 56) (width 0.3) (layer "F.Cu") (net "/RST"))
 (segment (start 76.5 60.5) (end 77.035 60.5) (width 0.3) (layer "F.Cu") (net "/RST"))
 (segment (start 77.035 60.5) (end 78.615 62.08) (width 0.3) (layer "F.Cu") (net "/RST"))
 (via (at 75.5 56) (size 0.6) (drill 0.3) (layers "F.Cu" "B.Cu") (capping no) (covering (front no) (back no))
  (plugging (front no) (back no)) (filling no) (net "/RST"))
 (via (at 76.5 60.5) (size 0.6) (drill 0.3) (layers "F.Cu" "B.Cu") (capping no) (covering (front no) (back no))
  (plugging (front no) (back no)) (filling no) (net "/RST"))
 (segment (start 75.5 56) (end 76.5 57) (width 0.3) (layer "B.Cu") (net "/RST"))
 (segment (start 76.5 57) (end 76.5 60.5) (width 0.3) (layer "B.Cu") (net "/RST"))
 (segment (start 67.5 54.5) (end 67 55) (width 0.3) (layer "F.Cu") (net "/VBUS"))
 (segment (start 63.599 56.581) (end 64.18 56) (width 0.3) (layer "F.Cu") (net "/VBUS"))
 (segment (start 63.599 57.919) (end 63.599 56.581) (width 0.3) (layer "F.Cu") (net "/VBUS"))
 (segment (start 61.86 57) (end 61.86 56.64) (width 0.3) (layer "F.Cu") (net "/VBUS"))
 (segment (start 67.55 54.55) (end 67.5 54.5) (width 0.3) (layer "F.Cu") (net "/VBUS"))
 (segment (start 76 54) (end 76.46 54.46) (width 0.2) (layer "F.Cu") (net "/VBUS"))
 (segment (start 66 54.5) (end 66.05 54.5) (width 0.3) (layer "F.Cu") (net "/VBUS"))
 (segment (start 58 60) (end 58.84 60) (width 0.3) (layer "F.Cu") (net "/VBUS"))
 (segment (start 67.05 55.5) (end 67 55.5) (width 0.3) (layer "F.Cu") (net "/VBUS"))
 (segment (start 63.5 55) (end 64.18 55) (width 0.3) (layer "F.Cu") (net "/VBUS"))
 (segment (start 54.969 54.749) (end 55.846 54.749) (width 0.3) (layer "F.Cu") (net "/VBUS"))
 (segment (start 57.45 59.45) (end 58 60) (width 0.3) (layer "F.Cu") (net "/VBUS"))
 (segment (start 76.46 54.46) (end 78.615 54.46) (width 0.2) (layer "F.Cu") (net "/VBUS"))
 (segment (start 64.18 55) (end 64.18 56) (width 0.3) (layer "F.Cu") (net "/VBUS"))
 (segment (start 59.491 59.349) (end 61.011 59.349) (width 0.3) (layer "F.Cu") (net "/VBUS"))
 (segment (start 67.05 55.5) (end 66.05 54.5) (width 0.3) (layer "F.Cu") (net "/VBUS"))
 (segment (start 61.011 59.349) (end 61.86 58.5) (width 0.3) (layer "F.Cu") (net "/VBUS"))
 (segment (start 58.84 60) (end 59.491 59.349) (width 0.3) (layer "F.Cu") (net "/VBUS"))
 (segment (start 54.5 55.218) (end 54.969 54.749) (width 0.3) (layer "F.Cu") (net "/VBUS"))
 (segment (start 63 55.5) (end 63.5 55) (width 0.3) (layer "F.Cu") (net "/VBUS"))
 (segment (start 55.846 54.749) (end 56.045 54.55) (width 0.3) (layer "F.Cu") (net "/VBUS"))
 (segment (start 56.045 59.45) (end 55.846 59.251) (width 0.3) (layer "F.Cu") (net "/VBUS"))
 (segment (start 67 55.5) (end 67 55) (width 0.3) (layer "F.Cu") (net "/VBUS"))
 (segment (start 74.5 54) (end 76 54) (width 0.2) (layer "F.Cu") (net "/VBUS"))
 (segment (start 68 54.55) (end 67.55 54.55) (width 0.3) (layer "F.Cu") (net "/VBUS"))
 (segment (start 63.599 57.919) (end 64.18 58.5) (width 0.3) (layer "F.Cu") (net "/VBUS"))
 (segment (start 61.86 58.5) (end 61.86 57) (width 0.3) (layer "F.Cu") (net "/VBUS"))
 (segment (start 55.846 59.251) (end 54.969 59.251) (width 0.3) (layer "F.Cu") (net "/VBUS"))
 (segment (start 54.969 59.251) (end 54.5 58.782) (width 0.3) (layer "F.Cu") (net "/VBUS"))
 (segment (start 54.5 58.782) (end 54.5 55.218) (width 0.3) (layer "F.Cu") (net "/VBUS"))
 (segment (start 61.86 56.64) (end 63 55.5) (width 0.3) (layer "F.Cu") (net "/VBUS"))
 (segment (start 63 55.5) (end 62.768 55.732) (width 0.3) (layer "F.Cu") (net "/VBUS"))
 (segment (start 56.045 59.45) (end 57.45 59.45) (width 0.3) (layer "F.Cu") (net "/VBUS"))
 (via (at 74.5 54) (size 0.6) (drill 0.3) (layers "F.Cu" "B.Cu") (capping no) (covering (front no) (back no))
  (plugging (front no) (back no)) (filling no) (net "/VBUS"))
 (via (at 62.75 55.75) (size 0.6) (drill 0.3) (layers "F.Cu" "B.Cu") (capping no) (covering (front no) (back no))
  (plugging (front no) (back no)) (filling no) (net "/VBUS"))
 (via (at 66.05 54.5) (size 0.6) (drill 0.3) (layers "F.Cu" "B.Cu") (capping no) (covering (front no) (back no))
  (plugging (front no) (back no)) (filling no) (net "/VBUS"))
 (segment (start 64.8 55.75) (end 66.05 54.5) (width 0.2) (layer "B.Cu") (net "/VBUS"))
 (segment (start 62.75 55.75) (end 64.8 55.75) (width 0.2) (layer "B.Cu") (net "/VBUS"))
 (segment (start 74.5 54) (end 66.55 54) (width 0.2) (layer "B.Cu") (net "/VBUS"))
 (segment (start 66.55 54) (end 66.05 54.5) (width 0.2) (layer "B.Cu") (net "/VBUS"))
 (segment (start 58.5 56.77302) (end 59.830096 56.77302) (width 0.2) (layer "F.Cu") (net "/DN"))
 (segment (start 69.475 54.525) (end 69.5 54.55) (width 0.2) (layer "F.Cu") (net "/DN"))
 (segment (start 57.132501 56.75) (end 57.155521 56.77302) (width 0.2) (layer "F.Cu") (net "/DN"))
 (segment (start 59 55.66) (end 59 56.27302) (width 0.2) (layer "F.Cu") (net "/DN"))
 (segment (start 64.106096 52.49702) (end 68.279832 52.49702) (width 0.2) (layer "F.Cu") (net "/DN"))
 (segment (start 69.475 53.692188) (end 69.475 54.525) (width 0.2) (layer "F.Cu") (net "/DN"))
 (segment (start 56.045 56.75) (end 57.132501 56.75) (width 0.2) (layer "F.Cu") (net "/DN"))
 (segment (start 59.830096 56.77302) (end 64.106096 52.49702) (width 0.2) (layer "F.Cu") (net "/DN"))
 (segment (start 58 56.77302) (end 58.5 56.77302) (width 0.2) (layer "F.Cu") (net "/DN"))
 (segment (start 68.279832 52.49702) (end 69.475 53.692188) (width 0.2) (layer "F.Cu") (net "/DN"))
 (segment (start 59 56.27302) (end 58.5 56.77302) (width 0.2) (layer "F.Cu") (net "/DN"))
 (segment (start 57.155521 56.77302) (end 58 56.77302) (width 0.2) (layer "F.Cu") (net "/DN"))
 (segment (start 68.092616 52.949) (end 69 53.856383) (width 0.2) (layer "F.Cu") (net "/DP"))
 (segment (start 64.293312 52.949) (end 68.092616 52.949) (width 0.2) (layer "F.Cu") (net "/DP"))
 (segment (start 56.045 57.25) (end 57.132501 57.25) (width 0.2) (layer "F.Cu") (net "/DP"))
 (segment (start 57.132501 57.25) (end 57.157501 57.225) (width 0.2) (layer "F.Cu") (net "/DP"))
 (segment (start 60.017312 57.225) (end 64.293312 52.949) (width 0.2) (layer "F.Cu") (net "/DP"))
 (segment (start 69 53.856383) (end 69 54.55) (width 0.2) (layer "F.Cu") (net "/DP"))
 (segment (start 57.157501 57.225) (end 60.017312 57.225) (width 0.2) (layer "F.Cu") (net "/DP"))
 (segment (start 64.82 59.129418) (end 64.18 59.769418) (width 0.3) (layer "F.Cu") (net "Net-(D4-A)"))
 (segment (start 64.18 59.769418) (end 64.18 60) (width 0.3) (layer "F.Cu") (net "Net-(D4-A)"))
 (segment (start 64.82 58.5) (end 64.82 59.129418) (width 0.3) (layer "F.Cu") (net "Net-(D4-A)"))
 (segment (start 72.68 56.5) (end 73.18 57) (width 0.3) (layer "F.Cu") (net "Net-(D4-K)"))
 (segment (start 71.95 56.5) (end 72.68 56.5) (width 0.3) (layer "F.Cu") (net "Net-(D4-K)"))
 (segment (start 71.5 61) (end 71.5 61.15) (width 0.3) (layer "F.Cu") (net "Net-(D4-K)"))
 (segment (start 73.68 56.68) (end 73.5 56.5) (width 0.3) (layer "F.Cu") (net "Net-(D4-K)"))
 (segment (start 65.97 61.15) (end 64.82 60) (width 0.3) (layer "F.Cu") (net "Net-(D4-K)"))
 (segment (start 73.68 57) (end 73.68 56.68) (width 0.3) (layer "F.Cu") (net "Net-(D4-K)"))
 (segment (start 71.5 61.15) (end 65.97 61.15) (width 0.3) (layer "F.Cu") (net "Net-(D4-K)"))
 (segment (start 73.18 57) (end 73.68 57) (width 0.3) (layer "F.Cu") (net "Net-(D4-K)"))
 (via (at 73.5 56.5) (size 0.6) (drill 0.3) (layers "F.Cu" "B.Cu") (capping no) (covering (front no) (back no))
  (plugging (front no) (back no)) (filling no) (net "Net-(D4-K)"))
 (via (at 71.5 61.15) (size 0.6) (drill 0.3) (layers "F.Cu" "B.Cu") (capping no) (covering (front no) (back no))
  (plugging (front no) (back no)) (filling no) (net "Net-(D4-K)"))
 (segment (start 73.5 56.5) (end 73 57) (width 0.3) (layer "B.Cu") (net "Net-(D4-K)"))
 (segment (start 73 57) (end 73 59.65) (width 0.3) (layer "B.Cu") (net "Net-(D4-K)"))
 (segment (start 73 59.65) (end 71.5 61.15) (width 0.3) (layer "B.Cu") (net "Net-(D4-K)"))
 (segment (start 64.18 56.870582) (end 64.82 56.230582) (width 0.3) (layer "F.Cu") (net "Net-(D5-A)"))
 (segment (start 64.18 57.5) (end 64.18 56.870582) (width 0.3) (layer "F.Cu") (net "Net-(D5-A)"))
 (segment (start 64.82 56.230582) (end 64.82 56) (width 0.3) (layer "F.Cu") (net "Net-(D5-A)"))
 (segment (start 72.550582 60.5) (end 73.68 59.370582) (width 0.3) (layer "F.Cu") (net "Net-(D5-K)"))
 (segment (start 73.68 58.24349) (end 73.68 58.5) (width 0.3) (layer "F.Cu") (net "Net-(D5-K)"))
 (segment (start 65.5 57.5) (end 64.82 57.5) (width 0.3) (layer "F.Cu") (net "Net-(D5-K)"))
 (segment (start 71.95 57) (end 72.43651 57) (width 0.3) (layer "F.Cu") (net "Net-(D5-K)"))
 (segment (start 73.68 58.5) (end 73.739 58.5) (width 0.3) (layer "F.Cu") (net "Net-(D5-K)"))
 (segment (start 66.5 60.5) (end 66 60) (width 0.3) (layer "F.Cu") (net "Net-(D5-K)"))
 (segment (start 72.550582 60.5) (end 66.5 60.5) (width 0.3) (layer "F.Cu") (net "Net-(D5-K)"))
 (segment (start 66 58) (end 65.5 57.5) (width 0.3) (layer "F.Cu") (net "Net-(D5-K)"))
 (segment (start 66 60) (end 66 58) (width 0.3) (layer "F.Cu") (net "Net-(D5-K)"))
 (segment (start 73.68 59.370582) (end 73.68 58.5) (width 0.3) (layer "F.Cu") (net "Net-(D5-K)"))
 (segment (start 72.43651 57) (end 73.68 58.24349) (width 0.3) (layer "F.Cu") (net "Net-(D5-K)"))
 (segment (start 56.045 55.75) (end 57.25 55.75) (width 0.2) (layer "F.Cu") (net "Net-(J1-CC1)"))
 (segment (start 57.5 55.5) (end 57.5 54) (width 0.2) (layer "F.Cu") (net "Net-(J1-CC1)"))
 (segment (start 57.25 55.75) (end 57.5 55.5) (width 0.2) (layer "F.Cu") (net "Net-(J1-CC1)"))
 (segment (start 57.5 54) (end 58.5 53) (width 0.2) (layer "F.Cu") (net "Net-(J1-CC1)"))
 (segment (start 56.045 58.75) (end 57.25 58.75) (width 0.3) (layer "F.Cu") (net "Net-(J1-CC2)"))
 (segment (start 57.25 58.75) (end 57.5 58.5) (width 0.3) (layer "F.Cu") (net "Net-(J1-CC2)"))
 (segment (start 57.5 58.5) (end 59.18 58.5) (width 0.3) (layer "F.Cu") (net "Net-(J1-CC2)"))
 (segment (start 74.5 57) (end 75.5 58) (width 0.3) (layer "F.Cu") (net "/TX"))
 (segment (start 75.5 59.5) (end 75.54 59.54) (width 0.3) (layer "F.Cu") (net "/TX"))
 (segment (start 75.5 58) (end 75.5 57.85) (width 0.3) (layer "F.Cu") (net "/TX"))
 (segment (start 75.54 59.54) (end 78.615 59.54) (width 0.3) (layer "F.Cu") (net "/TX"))
 (segment (start 74.32 57) (end 74.5 57) (width 0.3) (layer "F.Cu") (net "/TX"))
 (via (at 75.5 59.5) (size 0.6) (drill 0.3) (layers "F.Cu" "B.Cu") (capping no) (covering (front no) (back no))
  (plugging (front no) (back no)) (filling no) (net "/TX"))
 (via (at 75.5 57.85) (size 0.6) (drill 0.3) (layers "F.Cu" "B.Cu") (capping no) (covering (front no) (back no))
  (plugging (front no) (back no)) (filling no) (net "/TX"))
 (segment (start 75.5 57.85) (end 75.5 59.5) (width 0.3) (layer "B.Cu") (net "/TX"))
 (segment (start 74.32 58.5) (end 74.32 58.730582) (width 0.3) (layer "F.Cu") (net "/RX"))
 (segment (start 77.115 58.5) (end 78.615 57) (width 0.3) (layer "F.Cu") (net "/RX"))
 (segment (start 74.32 58.5) (end 77.115 58.5) (width 0.3) (layer "F.Cu") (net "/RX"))
 (segment (start 74.32 58.269418) (end 74.32 58.5) (width 0.3) (layer "F.Cu") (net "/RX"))
 (segment (start 65.821 56.001) (end 67.05 56.001) (width 0.3) (layer "F.Cu") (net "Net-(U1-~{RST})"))
 (segment (start 64.82 55) (end 65.821 56.001) (width 0.3) (layer "F.Cu") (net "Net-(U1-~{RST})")))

